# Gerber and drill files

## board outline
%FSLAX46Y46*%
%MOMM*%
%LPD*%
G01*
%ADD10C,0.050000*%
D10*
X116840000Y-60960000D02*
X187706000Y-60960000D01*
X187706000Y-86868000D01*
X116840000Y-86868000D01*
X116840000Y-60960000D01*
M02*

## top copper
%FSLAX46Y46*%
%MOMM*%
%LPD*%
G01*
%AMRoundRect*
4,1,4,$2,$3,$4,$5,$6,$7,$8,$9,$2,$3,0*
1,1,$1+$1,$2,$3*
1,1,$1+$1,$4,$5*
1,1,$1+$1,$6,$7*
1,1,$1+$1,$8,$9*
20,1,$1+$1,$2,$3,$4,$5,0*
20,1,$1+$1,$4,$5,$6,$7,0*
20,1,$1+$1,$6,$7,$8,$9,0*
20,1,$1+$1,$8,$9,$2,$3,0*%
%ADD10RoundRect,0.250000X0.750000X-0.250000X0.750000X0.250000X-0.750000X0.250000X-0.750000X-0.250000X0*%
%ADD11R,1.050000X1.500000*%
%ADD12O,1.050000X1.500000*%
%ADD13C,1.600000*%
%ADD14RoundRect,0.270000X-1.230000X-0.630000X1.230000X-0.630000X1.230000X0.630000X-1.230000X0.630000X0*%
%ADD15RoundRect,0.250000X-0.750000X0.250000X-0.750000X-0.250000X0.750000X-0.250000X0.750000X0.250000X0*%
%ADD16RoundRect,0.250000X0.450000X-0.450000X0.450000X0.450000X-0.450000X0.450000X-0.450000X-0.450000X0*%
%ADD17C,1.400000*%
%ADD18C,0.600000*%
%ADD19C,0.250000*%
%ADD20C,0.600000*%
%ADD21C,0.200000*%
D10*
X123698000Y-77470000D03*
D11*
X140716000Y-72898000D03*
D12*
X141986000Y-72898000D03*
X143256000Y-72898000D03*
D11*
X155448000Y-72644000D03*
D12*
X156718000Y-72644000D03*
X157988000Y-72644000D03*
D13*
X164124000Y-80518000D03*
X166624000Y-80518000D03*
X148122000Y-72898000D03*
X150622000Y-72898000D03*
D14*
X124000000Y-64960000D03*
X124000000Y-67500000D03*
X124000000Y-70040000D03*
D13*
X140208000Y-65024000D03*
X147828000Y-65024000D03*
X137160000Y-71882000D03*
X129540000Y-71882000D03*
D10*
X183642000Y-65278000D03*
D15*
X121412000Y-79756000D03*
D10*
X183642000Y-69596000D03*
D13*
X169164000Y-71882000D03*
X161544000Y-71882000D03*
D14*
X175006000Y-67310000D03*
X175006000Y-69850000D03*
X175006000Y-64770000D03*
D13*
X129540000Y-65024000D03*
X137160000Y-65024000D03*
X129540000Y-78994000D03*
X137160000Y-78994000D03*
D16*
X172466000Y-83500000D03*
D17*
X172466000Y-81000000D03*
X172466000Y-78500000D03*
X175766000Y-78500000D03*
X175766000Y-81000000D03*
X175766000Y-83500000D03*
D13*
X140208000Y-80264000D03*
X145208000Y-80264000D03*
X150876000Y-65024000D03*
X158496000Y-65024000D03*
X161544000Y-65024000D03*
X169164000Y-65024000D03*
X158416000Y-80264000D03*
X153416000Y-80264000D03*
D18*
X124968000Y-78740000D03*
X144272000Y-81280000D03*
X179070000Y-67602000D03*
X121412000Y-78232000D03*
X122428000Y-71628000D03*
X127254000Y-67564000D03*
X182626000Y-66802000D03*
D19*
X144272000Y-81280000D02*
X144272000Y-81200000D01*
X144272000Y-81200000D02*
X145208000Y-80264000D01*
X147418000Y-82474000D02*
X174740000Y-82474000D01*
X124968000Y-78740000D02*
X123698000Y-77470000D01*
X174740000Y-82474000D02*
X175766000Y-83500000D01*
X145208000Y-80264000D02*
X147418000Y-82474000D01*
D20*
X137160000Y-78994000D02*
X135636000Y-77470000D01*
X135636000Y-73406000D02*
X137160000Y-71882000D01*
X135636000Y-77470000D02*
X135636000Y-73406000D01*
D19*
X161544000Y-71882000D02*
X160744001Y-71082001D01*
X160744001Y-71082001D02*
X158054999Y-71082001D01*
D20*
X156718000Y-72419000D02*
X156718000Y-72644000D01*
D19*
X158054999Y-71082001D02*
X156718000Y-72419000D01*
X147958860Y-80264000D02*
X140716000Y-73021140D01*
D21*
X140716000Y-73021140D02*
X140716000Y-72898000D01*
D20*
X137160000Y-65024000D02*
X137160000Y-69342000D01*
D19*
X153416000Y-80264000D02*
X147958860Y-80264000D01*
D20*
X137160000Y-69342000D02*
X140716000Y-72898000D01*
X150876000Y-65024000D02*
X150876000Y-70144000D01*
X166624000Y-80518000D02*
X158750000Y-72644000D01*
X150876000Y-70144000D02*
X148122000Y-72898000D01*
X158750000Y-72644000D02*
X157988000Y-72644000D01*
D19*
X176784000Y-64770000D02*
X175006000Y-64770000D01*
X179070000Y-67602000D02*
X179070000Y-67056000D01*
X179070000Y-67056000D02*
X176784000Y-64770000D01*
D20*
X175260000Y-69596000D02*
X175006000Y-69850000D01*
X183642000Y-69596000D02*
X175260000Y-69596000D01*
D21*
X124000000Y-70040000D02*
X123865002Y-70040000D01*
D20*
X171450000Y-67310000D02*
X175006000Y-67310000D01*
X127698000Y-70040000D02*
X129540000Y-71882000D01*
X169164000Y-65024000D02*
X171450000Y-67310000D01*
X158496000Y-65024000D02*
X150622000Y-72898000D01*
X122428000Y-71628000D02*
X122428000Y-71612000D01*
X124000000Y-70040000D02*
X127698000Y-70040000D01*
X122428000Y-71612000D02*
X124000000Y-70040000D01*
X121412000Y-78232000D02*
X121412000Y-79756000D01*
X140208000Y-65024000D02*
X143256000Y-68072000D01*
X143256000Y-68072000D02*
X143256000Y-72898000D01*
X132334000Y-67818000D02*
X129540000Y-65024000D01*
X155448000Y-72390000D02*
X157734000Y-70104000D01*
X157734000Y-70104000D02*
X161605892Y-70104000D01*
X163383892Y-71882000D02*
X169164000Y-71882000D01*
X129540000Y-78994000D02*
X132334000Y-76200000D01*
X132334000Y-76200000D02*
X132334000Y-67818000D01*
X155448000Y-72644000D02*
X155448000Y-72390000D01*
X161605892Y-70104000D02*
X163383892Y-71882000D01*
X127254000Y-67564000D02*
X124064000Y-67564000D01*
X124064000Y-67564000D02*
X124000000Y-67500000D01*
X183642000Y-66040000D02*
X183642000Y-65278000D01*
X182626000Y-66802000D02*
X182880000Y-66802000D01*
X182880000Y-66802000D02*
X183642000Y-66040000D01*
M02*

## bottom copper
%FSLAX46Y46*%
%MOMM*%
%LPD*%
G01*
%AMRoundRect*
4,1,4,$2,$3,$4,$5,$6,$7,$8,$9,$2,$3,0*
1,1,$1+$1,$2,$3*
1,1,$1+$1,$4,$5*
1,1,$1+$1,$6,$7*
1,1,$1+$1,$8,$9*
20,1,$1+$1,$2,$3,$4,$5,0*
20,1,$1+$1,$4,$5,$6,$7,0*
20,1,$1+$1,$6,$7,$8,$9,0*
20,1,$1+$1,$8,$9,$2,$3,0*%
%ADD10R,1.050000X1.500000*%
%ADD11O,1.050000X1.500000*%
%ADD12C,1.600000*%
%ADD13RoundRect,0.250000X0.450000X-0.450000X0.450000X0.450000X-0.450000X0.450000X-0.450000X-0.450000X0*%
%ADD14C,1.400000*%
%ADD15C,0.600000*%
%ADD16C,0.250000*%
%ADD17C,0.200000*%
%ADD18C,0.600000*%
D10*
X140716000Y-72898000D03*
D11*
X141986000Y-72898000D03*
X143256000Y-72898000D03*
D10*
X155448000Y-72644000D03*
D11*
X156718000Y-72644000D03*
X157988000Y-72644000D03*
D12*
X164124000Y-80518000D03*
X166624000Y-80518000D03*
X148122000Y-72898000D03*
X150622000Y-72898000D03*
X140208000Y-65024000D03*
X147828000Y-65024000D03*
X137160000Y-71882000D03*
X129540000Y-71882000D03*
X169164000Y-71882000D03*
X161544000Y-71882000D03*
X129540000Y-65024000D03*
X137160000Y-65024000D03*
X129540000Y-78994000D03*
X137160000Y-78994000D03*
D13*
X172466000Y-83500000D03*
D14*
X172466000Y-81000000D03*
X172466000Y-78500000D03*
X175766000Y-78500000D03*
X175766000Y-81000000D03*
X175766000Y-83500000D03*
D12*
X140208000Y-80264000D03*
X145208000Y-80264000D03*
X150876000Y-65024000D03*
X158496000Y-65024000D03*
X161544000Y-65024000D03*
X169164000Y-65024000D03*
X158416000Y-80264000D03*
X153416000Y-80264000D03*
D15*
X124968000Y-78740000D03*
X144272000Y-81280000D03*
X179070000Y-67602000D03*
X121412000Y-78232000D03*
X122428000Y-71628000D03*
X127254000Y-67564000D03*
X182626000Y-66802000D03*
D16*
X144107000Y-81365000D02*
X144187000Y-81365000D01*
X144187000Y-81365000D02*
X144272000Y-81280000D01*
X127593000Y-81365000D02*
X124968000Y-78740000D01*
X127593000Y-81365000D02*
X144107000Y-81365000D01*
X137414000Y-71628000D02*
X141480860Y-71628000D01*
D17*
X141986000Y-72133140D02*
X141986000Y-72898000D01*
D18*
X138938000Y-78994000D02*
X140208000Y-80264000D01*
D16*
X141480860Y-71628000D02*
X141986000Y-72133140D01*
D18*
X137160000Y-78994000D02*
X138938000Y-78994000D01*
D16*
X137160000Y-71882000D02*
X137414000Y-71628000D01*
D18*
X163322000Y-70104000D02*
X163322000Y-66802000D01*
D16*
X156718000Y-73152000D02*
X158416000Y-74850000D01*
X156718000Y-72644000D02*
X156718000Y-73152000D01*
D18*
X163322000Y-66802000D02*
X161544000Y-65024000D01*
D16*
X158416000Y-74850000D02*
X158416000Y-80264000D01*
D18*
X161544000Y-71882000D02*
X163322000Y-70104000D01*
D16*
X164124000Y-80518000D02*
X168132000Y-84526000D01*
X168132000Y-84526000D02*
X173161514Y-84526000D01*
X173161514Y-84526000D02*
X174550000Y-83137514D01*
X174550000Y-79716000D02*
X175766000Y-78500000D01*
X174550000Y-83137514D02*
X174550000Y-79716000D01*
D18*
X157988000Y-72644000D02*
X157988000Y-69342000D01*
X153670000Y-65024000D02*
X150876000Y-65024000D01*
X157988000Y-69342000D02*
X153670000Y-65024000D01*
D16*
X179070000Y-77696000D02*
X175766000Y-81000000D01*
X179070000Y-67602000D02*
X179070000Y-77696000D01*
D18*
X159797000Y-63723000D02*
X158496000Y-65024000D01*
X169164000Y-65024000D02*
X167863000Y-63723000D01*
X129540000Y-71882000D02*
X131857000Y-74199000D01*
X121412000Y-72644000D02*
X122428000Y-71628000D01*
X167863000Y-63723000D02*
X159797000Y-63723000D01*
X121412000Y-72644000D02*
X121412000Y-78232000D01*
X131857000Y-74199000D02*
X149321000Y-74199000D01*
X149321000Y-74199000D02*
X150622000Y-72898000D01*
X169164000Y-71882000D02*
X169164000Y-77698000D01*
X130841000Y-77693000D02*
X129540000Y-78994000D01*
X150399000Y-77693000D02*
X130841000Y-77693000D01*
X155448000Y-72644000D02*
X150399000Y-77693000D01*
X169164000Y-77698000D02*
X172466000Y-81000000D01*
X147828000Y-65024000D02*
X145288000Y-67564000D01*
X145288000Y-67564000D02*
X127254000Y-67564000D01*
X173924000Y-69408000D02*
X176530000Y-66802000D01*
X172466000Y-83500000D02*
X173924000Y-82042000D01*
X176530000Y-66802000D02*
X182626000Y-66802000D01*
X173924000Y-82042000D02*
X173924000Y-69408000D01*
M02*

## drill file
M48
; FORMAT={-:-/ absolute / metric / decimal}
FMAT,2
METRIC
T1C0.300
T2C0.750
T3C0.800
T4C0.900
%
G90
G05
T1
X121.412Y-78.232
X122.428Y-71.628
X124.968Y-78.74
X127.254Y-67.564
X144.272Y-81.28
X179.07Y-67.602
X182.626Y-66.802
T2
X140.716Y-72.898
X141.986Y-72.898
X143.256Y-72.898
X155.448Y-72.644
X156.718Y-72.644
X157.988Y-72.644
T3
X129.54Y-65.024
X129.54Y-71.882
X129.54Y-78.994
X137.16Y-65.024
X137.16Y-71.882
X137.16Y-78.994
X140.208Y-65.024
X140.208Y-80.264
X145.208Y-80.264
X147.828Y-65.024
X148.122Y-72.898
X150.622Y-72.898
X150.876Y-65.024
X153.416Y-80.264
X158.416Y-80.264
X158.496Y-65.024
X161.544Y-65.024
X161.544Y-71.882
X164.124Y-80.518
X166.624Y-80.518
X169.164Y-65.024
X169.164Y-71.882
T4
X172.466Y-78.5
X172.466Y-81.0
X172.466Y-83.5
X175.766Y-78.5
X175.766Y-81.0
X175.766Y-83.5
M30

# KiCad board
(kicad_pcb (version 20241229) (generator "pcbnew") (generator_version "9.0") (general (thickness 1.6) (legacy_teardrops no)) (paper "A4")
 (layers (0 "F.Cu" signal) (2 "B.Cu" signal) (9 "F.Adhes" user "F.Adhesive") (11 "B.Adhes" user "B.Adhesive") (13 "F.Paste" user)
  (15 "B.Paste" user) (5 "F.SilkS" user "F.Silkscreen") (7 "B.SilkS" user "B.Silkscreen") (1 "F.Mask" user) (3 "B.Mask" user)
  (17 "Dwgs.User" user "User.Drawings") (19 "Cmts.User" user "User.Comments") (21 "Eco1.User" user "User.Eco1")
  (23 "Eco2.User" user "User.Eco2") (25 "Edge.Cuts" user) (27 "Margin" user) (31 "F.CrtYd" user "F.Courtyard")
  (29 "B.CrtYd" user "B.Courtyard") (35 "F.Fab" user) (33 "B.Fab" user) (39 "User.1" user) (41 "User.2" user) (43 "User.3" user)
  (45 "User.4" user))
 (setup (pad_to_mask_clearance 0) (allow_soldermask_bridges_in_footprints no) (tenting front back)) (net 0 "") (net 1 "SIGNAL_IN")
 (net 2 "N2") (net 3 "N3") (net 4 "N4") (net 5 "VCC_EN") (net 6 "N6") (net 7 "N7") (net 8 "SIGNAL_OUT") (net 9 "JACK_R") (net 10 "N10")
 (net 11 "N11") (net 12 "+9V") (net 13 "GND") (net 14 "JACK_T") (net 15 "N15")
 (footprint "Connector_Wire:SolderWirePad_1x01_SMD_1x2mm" (layer "F.Cu") (at 123.698 77.47 90)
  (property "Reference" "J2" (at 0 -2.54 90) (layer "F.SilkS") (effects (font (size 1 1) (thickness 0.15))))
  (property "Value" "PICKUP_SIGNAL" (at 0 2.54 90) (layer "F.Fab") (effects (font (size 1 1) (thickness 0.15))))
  (pad "1" smd roundrect (at 0 0 90) (size 1 2) (layers "F.Cu" "F.Mask" "F.Paste") (roundrect_rratio 0.25) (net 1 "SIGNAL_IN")))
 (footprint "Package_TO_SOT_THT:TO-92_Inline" (layer "F.Cu") (at 140.716 72.898)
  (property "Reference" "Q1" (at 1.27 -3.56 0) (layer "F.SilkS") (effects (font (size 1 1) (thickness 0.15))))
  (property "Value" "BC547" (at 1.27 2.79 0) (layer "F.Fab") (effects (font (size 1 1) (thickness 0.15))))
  (pad "1" thru_hole rect (at 0 0) (size 1.05 1.5) (drill 0.75) (layers "*.Cu" "*.Mask") (remove_unused_layers no) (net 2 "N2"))
  (pad "2" thru_hole oval (at 1.27 0) (size 1.05 1.5) (drill 0.75) (layers "*.Cu" "*.Mask") (remove_unused_layers no) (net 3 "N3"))
  (pad "3" thru_hole oval (at 2.54 0) (size 1.05 1.5) (drill 0.75) (layers "*.Cu" "*.Mask") (remove_unused_layers no) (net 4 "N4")))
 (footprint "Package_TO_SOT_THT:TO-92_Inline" (layer "F.Cu") (at 155.448 72.644)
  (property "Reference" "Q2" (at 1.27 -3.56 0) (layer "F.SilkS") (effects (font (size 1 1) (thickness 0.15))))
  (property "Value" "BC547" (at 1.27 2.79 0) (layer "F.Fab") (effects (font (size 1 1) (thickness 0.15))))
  (pad "1" thru_hole rect (at 0 0) (size 1.05 1.5) (drill 0.75) (layers "*.Cu" "*.Mask") (remove_unused_layers no) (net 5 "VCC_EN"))
  (pad "2" thru_hole oval (at 1.27 0) (size 1.05 1.5) (drill 0.75) (layers "*.Cu" "*.Mask") (remove_unused_layers no) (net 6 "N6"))
  (pad "3" thru_hole oval (at 2.54 0) (size 1.05 1.5) (drill 0.75) (layers "*.Cu" "*.Mask") (remove_unused_layers no) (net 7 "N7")))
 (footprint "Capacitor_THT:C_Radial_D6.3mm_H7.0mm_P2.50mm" (layer "F.Cu") (at 164.124 80.518)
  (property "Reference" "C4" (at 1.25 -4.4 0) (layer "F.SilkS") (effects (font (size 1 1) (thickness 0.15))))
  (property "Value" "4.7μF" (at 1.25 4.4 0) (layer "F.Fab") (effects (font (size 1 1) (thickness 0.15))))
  (pad "1" thru_hole circle (at 0 0) (size 1.6 1.6) (drill 0.8) (layers "*.Cu" "*.Mask") (remove_unused_layers no) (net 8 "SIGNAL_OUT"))
  (pad "2" thru_hole circle (at 2.5 0) (size 1.6 1.6) (drill 0.8) (layers "*.Cu" "*.Mask") (remove_unused_layers no) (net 7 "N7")))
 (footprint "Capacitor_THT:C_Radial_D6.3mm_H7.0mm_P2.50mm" (layer "F.Cu") (at 148.122 72.898)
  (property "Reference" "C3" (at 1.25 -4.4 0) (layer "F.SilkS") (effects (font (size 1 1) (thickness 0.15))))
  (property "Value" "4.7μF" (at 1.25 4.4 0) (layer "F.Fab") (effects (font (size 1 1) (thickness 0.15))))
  (pad "1" thru_hole circle (at 0 0) (size 1.6 1.6) (drill 0.8) (layers "*.Cu" "*.Mask") (remove_unused_layers no) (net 7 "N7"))
  (pad "2" thru_hole circle (at 2.5 0) (size 1.6 1.6) (drill 0.8) (layers "*.Cu" "*.Mask") (remove_unused_layers no) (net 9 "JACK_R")))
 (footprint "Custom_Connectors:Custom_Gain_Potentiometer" (layer "F.Cu") (at 124 72.58)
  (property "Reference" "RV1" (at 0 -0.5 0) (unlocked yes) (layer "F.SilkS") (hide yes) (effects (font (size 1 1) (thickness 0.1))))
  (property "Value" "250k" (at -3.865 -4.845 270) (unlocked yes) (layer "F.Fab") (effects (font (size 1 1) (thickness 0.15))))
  (pad "1" smd roundrect (at 0 -7.62) (size 3 1.8) (layers "F.Cu" "F.Mask" "F.Paste") (roundrect_rratio 0.15) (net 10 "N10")
   (thermal_bridge_angle 45))
  (pad "2" smd roundrect (at 0 -5.08) (size 3 1.8) (layers "F.Cu" "F.Mask" "F.Paste") (roundrect_rratio 0.15) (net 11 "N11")
   (thermal_bridge_angle 45))
  (pad "3" smd roundrect (at 0 -2.54) (size 3 1.8) (layers "F.Cu" "F.Mask" "F.Paste") (roundrect_rratio 0.15) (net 9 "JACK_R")
   (thermal_bridge_angle 45)))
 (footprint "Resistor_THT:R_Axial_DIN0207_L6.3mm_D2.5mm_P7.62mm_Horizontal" (layer "F.Cu") (at 140.208 65.024)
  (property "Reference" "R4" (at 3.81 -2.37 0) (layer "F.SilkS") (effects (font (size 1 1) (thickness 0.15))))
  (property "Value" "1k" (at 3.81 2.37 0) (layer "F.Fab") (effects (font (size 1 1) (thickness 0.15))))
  (pad "1" thru_hole circle (at 0 0) (size 1.6 1.6) (drill 0.8) (layers "*.Cu" "*.Mask") (remove_unused_layers no) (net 4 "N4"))
  (pad "2" thru_hole circle (at 7.62 0) (size 1.6 1.6) (drill 0.8) (layers "*.Cu" "*.Mask") (remove_unused_layers no) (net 11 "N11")))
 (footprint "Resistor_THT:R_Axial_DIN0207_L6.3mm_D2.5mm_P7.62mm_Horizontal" (layer "F.Cu") (at 137.16 71.882 180)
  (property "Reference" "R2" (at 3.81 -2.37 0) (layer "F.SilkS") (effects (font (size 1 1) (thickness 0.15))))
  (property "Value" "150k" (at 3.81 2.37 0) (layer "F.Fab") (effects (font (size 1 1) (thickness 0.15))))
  (pad "1" thru_hole circle (at 0 0 180) (size 1.6 1.6) (drill 0.8) (layers "*.Cu" "*.Mask") (remove_unused_layers no) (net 3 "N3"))
  (pad "2" thru_hole circle (at 7.62 0 180) (size 1.6 1.6) (drill 0.8) (layers "*.Cu" "*.Mask") (remove_unused_layers no) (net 9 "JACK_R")))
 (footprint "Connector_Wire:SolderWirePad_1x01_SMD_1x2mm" (layer "F.Cu") (at 183.642 65.278 90)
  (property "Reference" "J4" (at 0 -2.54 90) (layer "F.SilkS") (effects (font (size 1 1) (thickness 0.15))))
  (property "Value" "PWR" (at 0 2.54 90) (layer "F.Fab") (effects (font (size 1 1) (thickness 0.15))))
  (pad "1" smd roundrect (at 0 0 90) (size 1 2) (layers "F.Cu" "F.Mask" "F.Paste") (roundrect_rratio 0.25) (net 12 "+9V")))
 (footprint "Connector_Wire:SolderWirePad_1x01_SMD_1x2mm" (layer "F.Cu") (at 121.412 79.756 -90)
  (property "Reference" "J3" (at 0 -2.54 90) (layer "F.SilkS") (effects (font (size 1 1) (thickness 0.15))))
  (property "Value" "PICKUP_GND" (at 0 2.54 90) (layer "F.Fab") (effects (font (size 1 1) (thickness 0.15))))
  (pad "1" smd roundrect (at 0 0 270) (size 1 2) (layers "F.Cu" "F.Mask" "F.Paste") (roundrect_rratio 0.25) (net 9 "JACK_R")))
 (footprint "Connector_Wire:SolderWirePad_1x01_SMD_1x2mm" (layer "F.Cu") (at 183.642 69.596 90)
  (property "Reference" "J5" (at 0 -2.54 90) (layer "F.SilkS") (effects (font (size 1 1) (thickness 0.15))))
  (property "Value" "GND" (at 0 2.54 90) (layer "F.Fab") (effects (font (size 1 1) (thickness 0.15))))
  (pad "1" smd roundrect (at 0 0 90) (size 1 2) (layers "F.Cu" "F.Mask" "F.Paste") (roundrect_rratio 0.25) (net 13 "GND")))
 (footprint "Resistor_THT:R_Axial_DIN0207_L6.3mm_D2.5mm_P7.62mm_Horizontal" (layer "F.Cu") (at 169.164 71.882 180)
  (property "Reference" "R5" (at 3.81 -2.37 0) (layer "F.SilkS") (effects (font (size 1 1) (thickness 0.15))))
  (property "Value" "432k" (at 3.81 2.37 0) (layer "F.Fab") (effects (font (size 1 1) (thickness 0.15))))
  (pad "1" thru_hole circle (at 0 0 180) (size 1.6 1.6) (drill 0.8) (layers "*.Cu" "*.Mask") (remove_unused_layers no) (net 5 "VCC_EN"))
  (pad "2" thru_hole circle (at 7.62 0 180) (size 1.6 1.6) (drill 0.8) (layers "*.Cu" "*.Mask") (remove_unused_layers no) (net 6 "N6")))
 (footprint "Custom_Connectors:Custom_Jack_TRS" (layer "F.Cu") (at 175.006 72.39)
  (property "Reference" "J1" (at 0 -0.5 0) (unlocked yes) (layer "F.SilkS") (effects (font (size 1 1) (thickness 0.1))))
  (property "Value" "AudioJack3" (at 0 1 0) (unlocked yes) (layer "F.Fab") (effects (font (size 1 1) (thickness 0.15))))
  (pad "R" smd roundrect (at 0 -5.08) (size 3 1.8) (layers "F.Cu" "F.Mask" "F.Paste") (roundrect_rratio 0.15) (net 9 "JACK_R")
   (thermal_bridge_angle 45))
  (pad "S" smd roundrect (at 0 -2.54) (size 3 1.8) (layers "F.Cu" "F.Mask" "F.Paste") (roundrect_rratio 0.15) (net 13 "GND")
   (thermal_bridge_angle 45))
  (pad "T" smd roundrect (at 0 -7.62) (size 3 1.8) (layers "F.Cu" "F.Mask" "F.Paste") (roundrect_rratio 0.15) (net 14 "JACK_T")
   (thermal_bridge_angle 45)))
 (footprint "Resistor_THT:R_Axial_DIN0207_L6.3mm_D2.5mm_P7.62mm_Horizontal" (layer "F.Cu") (at 129.54 65.024)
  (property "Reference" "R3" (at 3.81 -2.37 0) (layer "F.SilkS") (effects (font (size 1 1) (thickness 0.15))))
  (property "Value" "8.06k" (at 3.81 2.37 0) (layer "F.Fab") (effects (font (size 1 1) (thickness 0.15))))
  (pad "1" thru_hole circle (at 0 0) (size 1.6 1.6) (drill 0.8) (layers "*.Cu" "*.Mask") (remove_unused_layers no) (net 5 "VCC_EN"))
  (pad "2" thru_hole circle (at 7.62 0) (size 1.6 1.6) (drill 0.8) (layers "*.Cu" "*.Mask") (remove_unused_layers no) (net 2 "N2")))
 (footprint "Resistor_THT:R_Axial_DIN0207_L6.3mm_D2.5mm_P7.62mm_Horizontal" (layer "F.Cu") (at 129.54 78.994)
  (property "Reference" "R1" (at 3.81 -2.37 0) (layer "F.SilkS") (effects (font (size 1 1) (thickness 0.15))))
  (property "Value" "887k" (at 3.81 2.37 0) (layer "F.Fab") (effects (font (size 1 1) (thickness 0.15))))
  (pad "1" thru_hole circle (at 0 0) (size 1.6 1.6) (drill 0.8) (layers "*.Cu" "*.Mask") (remove_unused_layers no) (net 5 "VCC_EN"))
  (pad "2" thru_hole circle (at 7.62 0) (size 1.6 1.6) (drill 0.8) (layers "*.Cu" "*.Mask") (remove_unused_layers no) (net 3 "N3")))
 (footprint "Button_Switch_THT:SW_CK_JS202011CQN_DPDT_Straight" (layer "F.Cu") (at 172.466 83.5 90)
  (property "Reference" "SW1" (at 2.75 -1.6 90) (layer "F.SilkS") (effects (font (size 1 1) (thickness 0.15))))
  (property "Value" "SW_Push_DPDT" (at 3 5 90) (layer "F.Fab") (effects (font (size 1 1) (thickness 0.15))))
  (pad "1" thru_hole roundrect (at 0 0 90) (size 1.4 1.4) (drill 0.9) (layers "*.Cu" "*.Mask") (remove_unused_layers no)
   (roundrect_rratio 0.1785714286) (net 12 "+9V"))
  (pad "2" thru_hole circle (at 2.5 0 90) (size 1.4 1.4) (drill 0.9) (layers "*.Cu" "*.Mask") (remove_unused_layers no) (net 5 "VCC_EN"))
  (pad "3" thru_hole circle (at 5 0 90) (size 1.4 1.4) (drill 0.9) (layers "*.Cu" "*.Mask") (remove_unused_layers no) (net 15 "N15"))
  (pad "4" thru_hole circle (at 5 3.3 90) (size 1.4 1.4) (drill 0.9) (layers "*.Cu" "*.Mask") (remove_unused_layers no) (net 8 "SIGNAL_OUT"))
  (pad "5" thru_hole circle (at 2.5 3.3 90) (size 1.4 1.4) (drill 0.9) (layers "*.Cu" "*.Mask") (remove_unused_layers no) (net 14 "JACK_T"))
  (pad "6" thru_hole circle (at 0 3.3 90) (size 1.4 1.4) (drill 0.9) (layers "*.Cu" "*.Mask") (remove_unused_layers no) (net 1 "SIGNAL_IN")))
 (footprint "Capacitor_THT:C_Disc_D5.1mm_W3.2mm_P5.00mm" (layer "F.Cu") (at 140.208 80.264)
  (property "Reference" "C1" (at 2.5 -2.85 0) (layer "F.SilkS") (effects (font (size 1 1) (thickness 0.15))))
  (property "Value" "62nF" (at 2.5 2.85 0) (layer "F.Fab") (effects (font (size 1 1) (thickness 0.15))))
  (pad "1" thru_hole circle (at 0 0) (size 1.6 1.6) (drill 0.8) (layers "*.Cu" "*.Mask") (remove_unused_layers no) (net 3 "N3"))
  (pad "2" thru_hole circle (at 5 0) (size 1.6 1.6) (drill 0.8) (layers "*.Cu" "*.Mask") (remove_unused_layers no) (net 1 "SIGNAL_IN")))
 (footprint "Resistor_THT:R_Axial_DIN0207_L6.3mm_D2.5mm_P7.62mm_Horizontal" (layer "F.Cu") (at 150.876 65.024)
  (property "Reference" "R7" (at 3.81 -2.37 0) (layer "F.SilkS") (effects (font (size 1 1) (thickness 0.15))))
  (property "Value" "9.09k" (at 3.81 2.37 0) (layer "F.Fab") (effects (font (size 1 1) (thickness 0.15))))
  (pad "1" thru_hole circle (at 0 0) (size 1.6 1.6) (drill 0.8) (layers "*.Cu" "*.Mask") (remove_unused_layers no) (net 7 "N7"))
  (pad "2" thru_hole circle (at 7.62 0) (size 1.6 1.6) (drill 0.8) (layers "*.Cu" "*.Mask") (remove_unused_layers no) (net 9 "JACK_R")))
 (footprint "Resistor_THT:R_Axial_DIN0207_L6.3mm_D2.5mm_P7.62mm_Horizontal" (layer "F.Cu") (at 161.544 65.024)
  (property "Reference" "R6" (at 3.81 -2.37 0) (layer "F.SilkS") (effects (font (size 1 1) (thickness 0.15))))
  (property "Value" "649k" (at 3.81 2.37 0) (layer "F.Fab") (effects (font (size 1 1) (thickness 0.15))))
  (pad "1" thru_hole circle (at 0 0) (size 1.6 1.6) (drill 0.8) (layers "*.Cu" "*.Mask") (remove_unused_layers no) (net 6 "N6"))
  (pad "2" thru_hole circle (at 7.62 0) (size 1.6 1.6) (drill 0.8) (layers "*.Cu" "*.Mask") (remove_unused_layers no) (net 9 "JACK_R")))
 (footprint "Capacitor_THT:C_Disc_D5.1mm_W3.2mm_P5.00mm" (layer "F.Cu") (at 158.416 80.264 180)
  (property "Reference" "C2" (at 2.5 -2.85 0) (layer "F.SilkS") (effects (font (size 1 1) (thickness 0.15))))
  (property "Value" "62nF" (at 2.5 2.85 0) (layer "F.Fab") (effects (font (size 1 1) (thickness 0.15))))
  (pad "1" thru_hole circle (at 0 0 180) (size 1.6 1.6) (drill 0.8) (layers "*.Cu" "*.Mask") (remove_unused_layers no) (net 6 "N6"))
  (pad "2" thru_hole circle (at 5 0 180) (size 1.6 1.6) (drill 0.8) (layers "*.Cu" "*.Mask") (remove_unused_layers no) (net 2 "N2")))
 (gr_rect (start 116.84 60.96) (end 187.706 86.868) (stroke (width 0.05) (type default)) (fill no) (layer "Edge.Cuts"))
 (segment (start 144.272 81.28) (end 144.272 81.2) (width 0.25) (layer "F.Cu") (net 1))
 (segment (start 144.272 81.2) (end 145.208 80.264) (width 0.25) (layer "F.Cu") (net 1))
 (segment (start 147.418 82.474) (end 174.74 82.474) (width 0.25) (layer "F.Cu") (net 1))
 (segment (start 124.968 78.74) (end 123.698 77.47) (width 0.25) (layer "F.Cu") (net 1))
 (segment (start 174.74 82.474) (end 175.766 83.5) (width 0.25) (layer "F.Cu") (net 1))
 (segment (start 145.208 80.264) (end 147.418 82.474) (width 0.25) (layer "F.Cu") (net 1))
 (via (at 124.968 78.74) (size 0.6) (drill 0.3) (layers "F.Cu" "B.Cu") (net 1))
 (via (at 144.272 81.28) (size 0.6) (drill 0.3) (layers "F.Cu" "B.Cu") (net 1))
 (segment (start 144.107 81.365) (end 144.187 81.365) (width 0.25) (layer "B.Cu") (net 1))
 (segment (start 144.187 81.365) (end 144.272 81.28) (width 0.25) (layer "B.Cu") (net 1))
 (segment (start 127.593 81.365) (end 124.968 78.74) (width 0.25) (layer "B.Cu") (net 1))
 (segment (start 127.593 81.365) (end 144.107 81.365) (width 0.25) (layer "B.Cu") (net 1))
 (segment (start 137.16 78.994) (end 135.636 77.47) (width 0.6) (layer "F.Cu") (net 3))
 (segment (start 135.636 73.406) (end 137.16 71.882) (width 0.6) (layer "F.Cu") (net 3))
 (segment (start 135.636 77.47) (end 135.636 73.406) (width 0.6) (layer "F.Cu") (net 3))
 (segment (start 137.414 71.628) (end 141.48086 71.628) (width 0.25) (layer "B.Cu") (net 3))
 (segment (start 141.986 72.13314) (end 141.986 72.898) (width 0.2) (layer "B.Cu") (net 3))
 (segment (start 138.938 78.994) (end 140.208 80.264) (width 0.6) (layer "B.Cu") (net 3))
 (segment (start 141.48086 71.628) (end 141.986 72.13314) (width 0.25) (layer "B.Cu") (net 3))
 (segment (start 137.16 78.994) (end 138.938 78.994) (width 0.6) (layer "B.Cu") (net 3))
 (segment (start 137.16 71.882) (end 137.414 71.628) (width 0.25) (layer "B.Cu") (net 3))
 (segment (start 161.544 71.882) (end 160.744001 71.082001) (width 0.25) (layer "F.Cu") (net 6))
 (segment (start 160.744001 71.082001) (end 158.054999 71.082001) (width 0.25) (layer "F.Cu") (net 6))
 (segment (start 156.718 72.419) (end 156.718 72.644) (width 0.6) (layer "F.Cu") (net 6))
 (segment (start 158.054999 71.082001) (end 156.718 72.419) (width 0.25) (layer "F.Cu") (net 6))
 (segment (start 163.322 70.104) (end 163.322 66.802) (width 0.6) (layer "B.Cu") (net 6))
 (segment (start 156.718 73.152) (end 158.416 74.85) (width 0.25) (layer "B.Cu") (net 6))
 (segment (start 156.718 72.644) (end 156.718 73.152) (width 0.25) (layer "B.Cu") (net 6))
 (segment (start 163.322 66.802) (end 161.544 65.024) (width 0.6) (layer "B.Cu") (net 6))
 (segment (start 158.416 74.85) (end 158.416 80.264) (width 0.25) (layer "B.Cu") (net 6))
 (segment (start 161.544 71.882) (end 163.322 70.104) (width 0.6) (layer "B.Cu") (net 6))
 (segment (start 147.95886 80.264) (end 140.716 73.02114) (width 0.25) (layer "F.Cu") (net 2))
 (segment (start 140.716 73.02114) (end 140.716 72.898) (width 0.2) (layer "F.Cu") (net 2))
 (segment (start 137.16 65.024) (end 137.16 69.342) (width 0.6) (layer "F.Cu") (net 2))
 (segment (start 153.416 80.264) (end 147.95886 80.264) (width 0.25) (layer "F.Cu") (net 2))
 (segment (start 137.16 69.342) (end 140.716 72.898) (width 0.6) (layer "F.Cu") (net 2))
 (segment (start 164.124 80.518) (end 168.132 84.526) (width 0.25) (layer "B.Cu") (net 8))
 (segment (start 168.132 84.526) (end 173.161514 84.526) (width 0.25) (layer "B.Cu") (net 8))
 (segment (start 173.161514 84.526) (end 174.55 83.137514) (width 0.25) (layer "B.Cu") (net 8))
 (segment (start 174.55 79.716) (end 175.766 78.5) (width 0.25) (layer "B.Cu") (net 8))
 (segment (start 174.55 83.137514) (end 174.55 79.716) (width 0.25) (layer "B.Cu") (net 8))
 (segment (start 150.876 65.024) (end 150.876 70.144) (width 0.6) (layer "F.Cu") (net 7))
 (segment (start 166.624 80.518) (end 158.75 72.644) (width 0.6) (layer "F.Cu") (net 7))
 (segment (start 150.876 70.144) (end 148.122 72.898) (width 0.6) (layer "F.Cu") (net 7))
 (segment (start 158.75 72.644) (end 157.988 72.644) (width 0.6) (layer "F.Cu") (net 7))
 (segment (start 157.988 72.644) (end 157.988 69.342) (width 0.6) (layer "B.Cu") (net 7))
 (segment (start 153.67 65.024) (end 150.876 65.024) (width 0.6) (layer "B.Cu") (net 7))
 (segment (start 157.988 69.342) (end 153.67 65.024) (width 0.6) (layer "B.Cu") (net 7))
 (segment (start 176.784 64.77) (end 175.006 64.77) (width 0.25) (layer "F.Cu") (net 14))
 (segment (start 179.07 67.602) (end 179.07 67.056) (width 0.25) (layer "F.Cu") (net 14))
 (segment (start 179.07 67.056) (end 176.784 64.77) (width 0.25) (layer "F.Cu") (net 14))
 (via (at 179.07 67.602) (size 0.6) (drill 0.3) (layers "F.Cu" "B.Cu") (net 14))
 (segment (start 179.07 77.696) (end 175.766 81) (width 0.25) (layer "B.Cu") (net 14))
 (segment (start 179.07 67.602) (end 179.07 77.696) (width 0.25) (layer "B.Cu") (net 14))
 (segment (start 175.26 69.596) (end 175.006 69.85) (width 0.6) (layer "F.Cu") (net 13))
 (segment (start 183.642 69.596) (end 175.26 69.596) (width 0.6) (layer "F.Cu") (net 13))
 (segment (start 124 70.04) (end 123.865002 70.04) (width 0.2) (layer "F.Cu") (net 9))
 (segment (start 171.45 67.31) (end 175.006 67.31) (width 0.6) (layer "F.Cu") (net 9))
 (segment (start 127.698 70.04) (end 129.54 71.882) (width 0.6) (layer "F.Cu") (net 9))
 (segment (start 169.164 65.024) (end 171.45 67.31) (width 0.6) (layer "F.Cu") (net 9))
 (segment (start 158.496 65.024) (end 150.622 72.898) (width 0.6) (layer "F.Cu") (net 9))
 (segment (start 122.428 71.628) (end 122.428 71.612) (width 0.6) (layer "F.Cu") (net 9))
 (segment (start 124 70.04) (end 127.698 70.04) (width 0.6) (layer "F.Cu") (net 9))
 (segment (start 122.428 71.612) (end 124 70.04) (width 0.6) (layer "F.Cu") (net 9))
 (segment (start 121.412 78.232) (end 121.412 79.756) (width 0.6) (layer "F.Cu") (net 9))
 (via (at 121.412 78.232) (size 0.6) (drill 0.3) (layers "F.Cu" "B.Cu") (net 9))
 (via (at 122.428 71.628) (size 0.6) (drill 0.3) (layers "F.Cu" "B.Cu") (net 9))
 (segment (start 159.797 63.723) (end 158.496 65.024) (width 0.6) (layer "B.Cu") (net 9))
 (segment (start 169.164 65.024) (end 167.863 63.723) (width 0.6) (layer "B.Cu") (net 9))
 (segment (start 129.54 71.882) (end 131.857 74.199) (width 0.6) (layer "B.Cu") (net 9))
 (segment (start 121.412 72.644) (end 122.428 71.628) (width 0.6) (layer "B.Cu") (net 9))
 (segment (start 167.863 63.723) (end 159.797 63.723) (width 0.6) (layer "B.Cu") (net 9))
 (segment (start 121.412 72.644) (end 121.412 78.232) (width 0.6) (layer "B.Cu") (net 9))
 (segment (start 131.857 74.199) (end 149.321 74.199) (width 0.6) (layer "B.Cu") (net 9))
 (segment (start 149.321 74.199) (end 150.622 72.898) (width 0.6) (layer "B.Cu") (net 9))
 (segment (start 140.208 65.024) (end 143.256 68.072) (width 0.6) (layer "F.Cu") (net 4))
 (segment (start 143.256 68.072) (end 143.256 72.898) (width 0.6) (layer "F.Cu") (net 4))
 (segment (start 132.334 67.818) (end 129.54 65.024) (width 0.6) (layer "F.Cu") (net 5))
 (segment (start 155.448 72.39) (end 157.734 70.104) (width 0.6) (layer "F.Cu") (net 5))
 (segment (start 157.734 70.104) (end 161.605892 70.104) (width 0.6) (layer "F.Cu") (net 5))
 (segment (start 163.383892 71.882) (end 169.164 71.882) (width 0.6) (layer "F.Cu") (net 5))
 (segment (start 129.54 78.994) (end 132.334 76.2) (width 0.6) (layer "F.Cu") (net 5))
 (segment (start 132.334 76.2) (end 132.334 67.818) (width 0.6) (layer "F.Cu") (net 5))
 (segment (start 155.448 72.644) (end 155.448 72.39) (width 0.6) (layer "F.Cu") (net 5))
 (segment (start 161.605892 70.104) (end 163.383892 71.882) (width 0.6) (layer "F.Cu") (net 5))
 (segment (start 169.164 71.882) (end 169.164 77.698) (width 0.6) (layer "B.Cu") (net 5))
 (segment (start 130.841 77.693) (end 129.54 78.994) (width 0.6) (layer "B.Cu") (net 5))
 (segment (start 150.399 77.693) (end 130.841 77.693) (width 0.6) (layer "B.Cu") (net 5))
 (segment (start 155.448 72.644) (end 150.399 77.693) (width 0.6) (layer "B.Cu") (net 5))
 (segment (start 169.164 77.698) (end 172.466 81) (width 0.6) (layer "B.Cu") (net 5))
 (segment (start 127.254 67.564) (end 124.064 67.564) (width 0.6) (layer "F.Cu") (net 11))
 (segment (start 124.064 67.564) (end 124 67.5) (width 0.6) (layer "F.Cu") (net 11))
 (via (at 127.254 67.564) (size 0.6) (drill 0.3) (layers "F.Cu" "B.Cu") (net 11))
 (segment (start 147.828 65.024) (end 145.288 67.564) (width 0.6) (layer "B.Cu") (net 11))
 (segment (start 145.288 67.564) (end 127.254 67.564) (width 0.6) (layer "B.Cu") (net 11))
 (segment (start 183.642 66.04) (end 183.642 65.278) (width 0.6) (layer "F.Cu") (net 12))
 (segment (start 182.626 66.802) (end 182.88 66.802) (width 0.6) (layer "F.Cu") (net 12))
 (segment (start 182.88 66.802) (end 183.642 66.04) (width 0.6) (layer "F.Cu") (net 12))
 (via (at 182.626 66.802) (size 0.6) (drill 0.3) (layers "F.Cu" "B.Cu") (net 12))
 (segment (start 173.924 69.408) (end 176.53 66.802) (width 0.6) (layer "B.Cu") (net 12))
 (segment (start 172.466 83.5) (end 173.924 82.042) (width 0.6) (layer "B.Cu") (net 12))
 (segment (start 176.53 66.802) (end 182.626 66.802) (width 0.6) (layer "B.Cu") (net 12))
 (segment (start 173.924 82.042) (end 173.924 69.408) (width 0.6) (layer "B.Cu") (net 12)))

